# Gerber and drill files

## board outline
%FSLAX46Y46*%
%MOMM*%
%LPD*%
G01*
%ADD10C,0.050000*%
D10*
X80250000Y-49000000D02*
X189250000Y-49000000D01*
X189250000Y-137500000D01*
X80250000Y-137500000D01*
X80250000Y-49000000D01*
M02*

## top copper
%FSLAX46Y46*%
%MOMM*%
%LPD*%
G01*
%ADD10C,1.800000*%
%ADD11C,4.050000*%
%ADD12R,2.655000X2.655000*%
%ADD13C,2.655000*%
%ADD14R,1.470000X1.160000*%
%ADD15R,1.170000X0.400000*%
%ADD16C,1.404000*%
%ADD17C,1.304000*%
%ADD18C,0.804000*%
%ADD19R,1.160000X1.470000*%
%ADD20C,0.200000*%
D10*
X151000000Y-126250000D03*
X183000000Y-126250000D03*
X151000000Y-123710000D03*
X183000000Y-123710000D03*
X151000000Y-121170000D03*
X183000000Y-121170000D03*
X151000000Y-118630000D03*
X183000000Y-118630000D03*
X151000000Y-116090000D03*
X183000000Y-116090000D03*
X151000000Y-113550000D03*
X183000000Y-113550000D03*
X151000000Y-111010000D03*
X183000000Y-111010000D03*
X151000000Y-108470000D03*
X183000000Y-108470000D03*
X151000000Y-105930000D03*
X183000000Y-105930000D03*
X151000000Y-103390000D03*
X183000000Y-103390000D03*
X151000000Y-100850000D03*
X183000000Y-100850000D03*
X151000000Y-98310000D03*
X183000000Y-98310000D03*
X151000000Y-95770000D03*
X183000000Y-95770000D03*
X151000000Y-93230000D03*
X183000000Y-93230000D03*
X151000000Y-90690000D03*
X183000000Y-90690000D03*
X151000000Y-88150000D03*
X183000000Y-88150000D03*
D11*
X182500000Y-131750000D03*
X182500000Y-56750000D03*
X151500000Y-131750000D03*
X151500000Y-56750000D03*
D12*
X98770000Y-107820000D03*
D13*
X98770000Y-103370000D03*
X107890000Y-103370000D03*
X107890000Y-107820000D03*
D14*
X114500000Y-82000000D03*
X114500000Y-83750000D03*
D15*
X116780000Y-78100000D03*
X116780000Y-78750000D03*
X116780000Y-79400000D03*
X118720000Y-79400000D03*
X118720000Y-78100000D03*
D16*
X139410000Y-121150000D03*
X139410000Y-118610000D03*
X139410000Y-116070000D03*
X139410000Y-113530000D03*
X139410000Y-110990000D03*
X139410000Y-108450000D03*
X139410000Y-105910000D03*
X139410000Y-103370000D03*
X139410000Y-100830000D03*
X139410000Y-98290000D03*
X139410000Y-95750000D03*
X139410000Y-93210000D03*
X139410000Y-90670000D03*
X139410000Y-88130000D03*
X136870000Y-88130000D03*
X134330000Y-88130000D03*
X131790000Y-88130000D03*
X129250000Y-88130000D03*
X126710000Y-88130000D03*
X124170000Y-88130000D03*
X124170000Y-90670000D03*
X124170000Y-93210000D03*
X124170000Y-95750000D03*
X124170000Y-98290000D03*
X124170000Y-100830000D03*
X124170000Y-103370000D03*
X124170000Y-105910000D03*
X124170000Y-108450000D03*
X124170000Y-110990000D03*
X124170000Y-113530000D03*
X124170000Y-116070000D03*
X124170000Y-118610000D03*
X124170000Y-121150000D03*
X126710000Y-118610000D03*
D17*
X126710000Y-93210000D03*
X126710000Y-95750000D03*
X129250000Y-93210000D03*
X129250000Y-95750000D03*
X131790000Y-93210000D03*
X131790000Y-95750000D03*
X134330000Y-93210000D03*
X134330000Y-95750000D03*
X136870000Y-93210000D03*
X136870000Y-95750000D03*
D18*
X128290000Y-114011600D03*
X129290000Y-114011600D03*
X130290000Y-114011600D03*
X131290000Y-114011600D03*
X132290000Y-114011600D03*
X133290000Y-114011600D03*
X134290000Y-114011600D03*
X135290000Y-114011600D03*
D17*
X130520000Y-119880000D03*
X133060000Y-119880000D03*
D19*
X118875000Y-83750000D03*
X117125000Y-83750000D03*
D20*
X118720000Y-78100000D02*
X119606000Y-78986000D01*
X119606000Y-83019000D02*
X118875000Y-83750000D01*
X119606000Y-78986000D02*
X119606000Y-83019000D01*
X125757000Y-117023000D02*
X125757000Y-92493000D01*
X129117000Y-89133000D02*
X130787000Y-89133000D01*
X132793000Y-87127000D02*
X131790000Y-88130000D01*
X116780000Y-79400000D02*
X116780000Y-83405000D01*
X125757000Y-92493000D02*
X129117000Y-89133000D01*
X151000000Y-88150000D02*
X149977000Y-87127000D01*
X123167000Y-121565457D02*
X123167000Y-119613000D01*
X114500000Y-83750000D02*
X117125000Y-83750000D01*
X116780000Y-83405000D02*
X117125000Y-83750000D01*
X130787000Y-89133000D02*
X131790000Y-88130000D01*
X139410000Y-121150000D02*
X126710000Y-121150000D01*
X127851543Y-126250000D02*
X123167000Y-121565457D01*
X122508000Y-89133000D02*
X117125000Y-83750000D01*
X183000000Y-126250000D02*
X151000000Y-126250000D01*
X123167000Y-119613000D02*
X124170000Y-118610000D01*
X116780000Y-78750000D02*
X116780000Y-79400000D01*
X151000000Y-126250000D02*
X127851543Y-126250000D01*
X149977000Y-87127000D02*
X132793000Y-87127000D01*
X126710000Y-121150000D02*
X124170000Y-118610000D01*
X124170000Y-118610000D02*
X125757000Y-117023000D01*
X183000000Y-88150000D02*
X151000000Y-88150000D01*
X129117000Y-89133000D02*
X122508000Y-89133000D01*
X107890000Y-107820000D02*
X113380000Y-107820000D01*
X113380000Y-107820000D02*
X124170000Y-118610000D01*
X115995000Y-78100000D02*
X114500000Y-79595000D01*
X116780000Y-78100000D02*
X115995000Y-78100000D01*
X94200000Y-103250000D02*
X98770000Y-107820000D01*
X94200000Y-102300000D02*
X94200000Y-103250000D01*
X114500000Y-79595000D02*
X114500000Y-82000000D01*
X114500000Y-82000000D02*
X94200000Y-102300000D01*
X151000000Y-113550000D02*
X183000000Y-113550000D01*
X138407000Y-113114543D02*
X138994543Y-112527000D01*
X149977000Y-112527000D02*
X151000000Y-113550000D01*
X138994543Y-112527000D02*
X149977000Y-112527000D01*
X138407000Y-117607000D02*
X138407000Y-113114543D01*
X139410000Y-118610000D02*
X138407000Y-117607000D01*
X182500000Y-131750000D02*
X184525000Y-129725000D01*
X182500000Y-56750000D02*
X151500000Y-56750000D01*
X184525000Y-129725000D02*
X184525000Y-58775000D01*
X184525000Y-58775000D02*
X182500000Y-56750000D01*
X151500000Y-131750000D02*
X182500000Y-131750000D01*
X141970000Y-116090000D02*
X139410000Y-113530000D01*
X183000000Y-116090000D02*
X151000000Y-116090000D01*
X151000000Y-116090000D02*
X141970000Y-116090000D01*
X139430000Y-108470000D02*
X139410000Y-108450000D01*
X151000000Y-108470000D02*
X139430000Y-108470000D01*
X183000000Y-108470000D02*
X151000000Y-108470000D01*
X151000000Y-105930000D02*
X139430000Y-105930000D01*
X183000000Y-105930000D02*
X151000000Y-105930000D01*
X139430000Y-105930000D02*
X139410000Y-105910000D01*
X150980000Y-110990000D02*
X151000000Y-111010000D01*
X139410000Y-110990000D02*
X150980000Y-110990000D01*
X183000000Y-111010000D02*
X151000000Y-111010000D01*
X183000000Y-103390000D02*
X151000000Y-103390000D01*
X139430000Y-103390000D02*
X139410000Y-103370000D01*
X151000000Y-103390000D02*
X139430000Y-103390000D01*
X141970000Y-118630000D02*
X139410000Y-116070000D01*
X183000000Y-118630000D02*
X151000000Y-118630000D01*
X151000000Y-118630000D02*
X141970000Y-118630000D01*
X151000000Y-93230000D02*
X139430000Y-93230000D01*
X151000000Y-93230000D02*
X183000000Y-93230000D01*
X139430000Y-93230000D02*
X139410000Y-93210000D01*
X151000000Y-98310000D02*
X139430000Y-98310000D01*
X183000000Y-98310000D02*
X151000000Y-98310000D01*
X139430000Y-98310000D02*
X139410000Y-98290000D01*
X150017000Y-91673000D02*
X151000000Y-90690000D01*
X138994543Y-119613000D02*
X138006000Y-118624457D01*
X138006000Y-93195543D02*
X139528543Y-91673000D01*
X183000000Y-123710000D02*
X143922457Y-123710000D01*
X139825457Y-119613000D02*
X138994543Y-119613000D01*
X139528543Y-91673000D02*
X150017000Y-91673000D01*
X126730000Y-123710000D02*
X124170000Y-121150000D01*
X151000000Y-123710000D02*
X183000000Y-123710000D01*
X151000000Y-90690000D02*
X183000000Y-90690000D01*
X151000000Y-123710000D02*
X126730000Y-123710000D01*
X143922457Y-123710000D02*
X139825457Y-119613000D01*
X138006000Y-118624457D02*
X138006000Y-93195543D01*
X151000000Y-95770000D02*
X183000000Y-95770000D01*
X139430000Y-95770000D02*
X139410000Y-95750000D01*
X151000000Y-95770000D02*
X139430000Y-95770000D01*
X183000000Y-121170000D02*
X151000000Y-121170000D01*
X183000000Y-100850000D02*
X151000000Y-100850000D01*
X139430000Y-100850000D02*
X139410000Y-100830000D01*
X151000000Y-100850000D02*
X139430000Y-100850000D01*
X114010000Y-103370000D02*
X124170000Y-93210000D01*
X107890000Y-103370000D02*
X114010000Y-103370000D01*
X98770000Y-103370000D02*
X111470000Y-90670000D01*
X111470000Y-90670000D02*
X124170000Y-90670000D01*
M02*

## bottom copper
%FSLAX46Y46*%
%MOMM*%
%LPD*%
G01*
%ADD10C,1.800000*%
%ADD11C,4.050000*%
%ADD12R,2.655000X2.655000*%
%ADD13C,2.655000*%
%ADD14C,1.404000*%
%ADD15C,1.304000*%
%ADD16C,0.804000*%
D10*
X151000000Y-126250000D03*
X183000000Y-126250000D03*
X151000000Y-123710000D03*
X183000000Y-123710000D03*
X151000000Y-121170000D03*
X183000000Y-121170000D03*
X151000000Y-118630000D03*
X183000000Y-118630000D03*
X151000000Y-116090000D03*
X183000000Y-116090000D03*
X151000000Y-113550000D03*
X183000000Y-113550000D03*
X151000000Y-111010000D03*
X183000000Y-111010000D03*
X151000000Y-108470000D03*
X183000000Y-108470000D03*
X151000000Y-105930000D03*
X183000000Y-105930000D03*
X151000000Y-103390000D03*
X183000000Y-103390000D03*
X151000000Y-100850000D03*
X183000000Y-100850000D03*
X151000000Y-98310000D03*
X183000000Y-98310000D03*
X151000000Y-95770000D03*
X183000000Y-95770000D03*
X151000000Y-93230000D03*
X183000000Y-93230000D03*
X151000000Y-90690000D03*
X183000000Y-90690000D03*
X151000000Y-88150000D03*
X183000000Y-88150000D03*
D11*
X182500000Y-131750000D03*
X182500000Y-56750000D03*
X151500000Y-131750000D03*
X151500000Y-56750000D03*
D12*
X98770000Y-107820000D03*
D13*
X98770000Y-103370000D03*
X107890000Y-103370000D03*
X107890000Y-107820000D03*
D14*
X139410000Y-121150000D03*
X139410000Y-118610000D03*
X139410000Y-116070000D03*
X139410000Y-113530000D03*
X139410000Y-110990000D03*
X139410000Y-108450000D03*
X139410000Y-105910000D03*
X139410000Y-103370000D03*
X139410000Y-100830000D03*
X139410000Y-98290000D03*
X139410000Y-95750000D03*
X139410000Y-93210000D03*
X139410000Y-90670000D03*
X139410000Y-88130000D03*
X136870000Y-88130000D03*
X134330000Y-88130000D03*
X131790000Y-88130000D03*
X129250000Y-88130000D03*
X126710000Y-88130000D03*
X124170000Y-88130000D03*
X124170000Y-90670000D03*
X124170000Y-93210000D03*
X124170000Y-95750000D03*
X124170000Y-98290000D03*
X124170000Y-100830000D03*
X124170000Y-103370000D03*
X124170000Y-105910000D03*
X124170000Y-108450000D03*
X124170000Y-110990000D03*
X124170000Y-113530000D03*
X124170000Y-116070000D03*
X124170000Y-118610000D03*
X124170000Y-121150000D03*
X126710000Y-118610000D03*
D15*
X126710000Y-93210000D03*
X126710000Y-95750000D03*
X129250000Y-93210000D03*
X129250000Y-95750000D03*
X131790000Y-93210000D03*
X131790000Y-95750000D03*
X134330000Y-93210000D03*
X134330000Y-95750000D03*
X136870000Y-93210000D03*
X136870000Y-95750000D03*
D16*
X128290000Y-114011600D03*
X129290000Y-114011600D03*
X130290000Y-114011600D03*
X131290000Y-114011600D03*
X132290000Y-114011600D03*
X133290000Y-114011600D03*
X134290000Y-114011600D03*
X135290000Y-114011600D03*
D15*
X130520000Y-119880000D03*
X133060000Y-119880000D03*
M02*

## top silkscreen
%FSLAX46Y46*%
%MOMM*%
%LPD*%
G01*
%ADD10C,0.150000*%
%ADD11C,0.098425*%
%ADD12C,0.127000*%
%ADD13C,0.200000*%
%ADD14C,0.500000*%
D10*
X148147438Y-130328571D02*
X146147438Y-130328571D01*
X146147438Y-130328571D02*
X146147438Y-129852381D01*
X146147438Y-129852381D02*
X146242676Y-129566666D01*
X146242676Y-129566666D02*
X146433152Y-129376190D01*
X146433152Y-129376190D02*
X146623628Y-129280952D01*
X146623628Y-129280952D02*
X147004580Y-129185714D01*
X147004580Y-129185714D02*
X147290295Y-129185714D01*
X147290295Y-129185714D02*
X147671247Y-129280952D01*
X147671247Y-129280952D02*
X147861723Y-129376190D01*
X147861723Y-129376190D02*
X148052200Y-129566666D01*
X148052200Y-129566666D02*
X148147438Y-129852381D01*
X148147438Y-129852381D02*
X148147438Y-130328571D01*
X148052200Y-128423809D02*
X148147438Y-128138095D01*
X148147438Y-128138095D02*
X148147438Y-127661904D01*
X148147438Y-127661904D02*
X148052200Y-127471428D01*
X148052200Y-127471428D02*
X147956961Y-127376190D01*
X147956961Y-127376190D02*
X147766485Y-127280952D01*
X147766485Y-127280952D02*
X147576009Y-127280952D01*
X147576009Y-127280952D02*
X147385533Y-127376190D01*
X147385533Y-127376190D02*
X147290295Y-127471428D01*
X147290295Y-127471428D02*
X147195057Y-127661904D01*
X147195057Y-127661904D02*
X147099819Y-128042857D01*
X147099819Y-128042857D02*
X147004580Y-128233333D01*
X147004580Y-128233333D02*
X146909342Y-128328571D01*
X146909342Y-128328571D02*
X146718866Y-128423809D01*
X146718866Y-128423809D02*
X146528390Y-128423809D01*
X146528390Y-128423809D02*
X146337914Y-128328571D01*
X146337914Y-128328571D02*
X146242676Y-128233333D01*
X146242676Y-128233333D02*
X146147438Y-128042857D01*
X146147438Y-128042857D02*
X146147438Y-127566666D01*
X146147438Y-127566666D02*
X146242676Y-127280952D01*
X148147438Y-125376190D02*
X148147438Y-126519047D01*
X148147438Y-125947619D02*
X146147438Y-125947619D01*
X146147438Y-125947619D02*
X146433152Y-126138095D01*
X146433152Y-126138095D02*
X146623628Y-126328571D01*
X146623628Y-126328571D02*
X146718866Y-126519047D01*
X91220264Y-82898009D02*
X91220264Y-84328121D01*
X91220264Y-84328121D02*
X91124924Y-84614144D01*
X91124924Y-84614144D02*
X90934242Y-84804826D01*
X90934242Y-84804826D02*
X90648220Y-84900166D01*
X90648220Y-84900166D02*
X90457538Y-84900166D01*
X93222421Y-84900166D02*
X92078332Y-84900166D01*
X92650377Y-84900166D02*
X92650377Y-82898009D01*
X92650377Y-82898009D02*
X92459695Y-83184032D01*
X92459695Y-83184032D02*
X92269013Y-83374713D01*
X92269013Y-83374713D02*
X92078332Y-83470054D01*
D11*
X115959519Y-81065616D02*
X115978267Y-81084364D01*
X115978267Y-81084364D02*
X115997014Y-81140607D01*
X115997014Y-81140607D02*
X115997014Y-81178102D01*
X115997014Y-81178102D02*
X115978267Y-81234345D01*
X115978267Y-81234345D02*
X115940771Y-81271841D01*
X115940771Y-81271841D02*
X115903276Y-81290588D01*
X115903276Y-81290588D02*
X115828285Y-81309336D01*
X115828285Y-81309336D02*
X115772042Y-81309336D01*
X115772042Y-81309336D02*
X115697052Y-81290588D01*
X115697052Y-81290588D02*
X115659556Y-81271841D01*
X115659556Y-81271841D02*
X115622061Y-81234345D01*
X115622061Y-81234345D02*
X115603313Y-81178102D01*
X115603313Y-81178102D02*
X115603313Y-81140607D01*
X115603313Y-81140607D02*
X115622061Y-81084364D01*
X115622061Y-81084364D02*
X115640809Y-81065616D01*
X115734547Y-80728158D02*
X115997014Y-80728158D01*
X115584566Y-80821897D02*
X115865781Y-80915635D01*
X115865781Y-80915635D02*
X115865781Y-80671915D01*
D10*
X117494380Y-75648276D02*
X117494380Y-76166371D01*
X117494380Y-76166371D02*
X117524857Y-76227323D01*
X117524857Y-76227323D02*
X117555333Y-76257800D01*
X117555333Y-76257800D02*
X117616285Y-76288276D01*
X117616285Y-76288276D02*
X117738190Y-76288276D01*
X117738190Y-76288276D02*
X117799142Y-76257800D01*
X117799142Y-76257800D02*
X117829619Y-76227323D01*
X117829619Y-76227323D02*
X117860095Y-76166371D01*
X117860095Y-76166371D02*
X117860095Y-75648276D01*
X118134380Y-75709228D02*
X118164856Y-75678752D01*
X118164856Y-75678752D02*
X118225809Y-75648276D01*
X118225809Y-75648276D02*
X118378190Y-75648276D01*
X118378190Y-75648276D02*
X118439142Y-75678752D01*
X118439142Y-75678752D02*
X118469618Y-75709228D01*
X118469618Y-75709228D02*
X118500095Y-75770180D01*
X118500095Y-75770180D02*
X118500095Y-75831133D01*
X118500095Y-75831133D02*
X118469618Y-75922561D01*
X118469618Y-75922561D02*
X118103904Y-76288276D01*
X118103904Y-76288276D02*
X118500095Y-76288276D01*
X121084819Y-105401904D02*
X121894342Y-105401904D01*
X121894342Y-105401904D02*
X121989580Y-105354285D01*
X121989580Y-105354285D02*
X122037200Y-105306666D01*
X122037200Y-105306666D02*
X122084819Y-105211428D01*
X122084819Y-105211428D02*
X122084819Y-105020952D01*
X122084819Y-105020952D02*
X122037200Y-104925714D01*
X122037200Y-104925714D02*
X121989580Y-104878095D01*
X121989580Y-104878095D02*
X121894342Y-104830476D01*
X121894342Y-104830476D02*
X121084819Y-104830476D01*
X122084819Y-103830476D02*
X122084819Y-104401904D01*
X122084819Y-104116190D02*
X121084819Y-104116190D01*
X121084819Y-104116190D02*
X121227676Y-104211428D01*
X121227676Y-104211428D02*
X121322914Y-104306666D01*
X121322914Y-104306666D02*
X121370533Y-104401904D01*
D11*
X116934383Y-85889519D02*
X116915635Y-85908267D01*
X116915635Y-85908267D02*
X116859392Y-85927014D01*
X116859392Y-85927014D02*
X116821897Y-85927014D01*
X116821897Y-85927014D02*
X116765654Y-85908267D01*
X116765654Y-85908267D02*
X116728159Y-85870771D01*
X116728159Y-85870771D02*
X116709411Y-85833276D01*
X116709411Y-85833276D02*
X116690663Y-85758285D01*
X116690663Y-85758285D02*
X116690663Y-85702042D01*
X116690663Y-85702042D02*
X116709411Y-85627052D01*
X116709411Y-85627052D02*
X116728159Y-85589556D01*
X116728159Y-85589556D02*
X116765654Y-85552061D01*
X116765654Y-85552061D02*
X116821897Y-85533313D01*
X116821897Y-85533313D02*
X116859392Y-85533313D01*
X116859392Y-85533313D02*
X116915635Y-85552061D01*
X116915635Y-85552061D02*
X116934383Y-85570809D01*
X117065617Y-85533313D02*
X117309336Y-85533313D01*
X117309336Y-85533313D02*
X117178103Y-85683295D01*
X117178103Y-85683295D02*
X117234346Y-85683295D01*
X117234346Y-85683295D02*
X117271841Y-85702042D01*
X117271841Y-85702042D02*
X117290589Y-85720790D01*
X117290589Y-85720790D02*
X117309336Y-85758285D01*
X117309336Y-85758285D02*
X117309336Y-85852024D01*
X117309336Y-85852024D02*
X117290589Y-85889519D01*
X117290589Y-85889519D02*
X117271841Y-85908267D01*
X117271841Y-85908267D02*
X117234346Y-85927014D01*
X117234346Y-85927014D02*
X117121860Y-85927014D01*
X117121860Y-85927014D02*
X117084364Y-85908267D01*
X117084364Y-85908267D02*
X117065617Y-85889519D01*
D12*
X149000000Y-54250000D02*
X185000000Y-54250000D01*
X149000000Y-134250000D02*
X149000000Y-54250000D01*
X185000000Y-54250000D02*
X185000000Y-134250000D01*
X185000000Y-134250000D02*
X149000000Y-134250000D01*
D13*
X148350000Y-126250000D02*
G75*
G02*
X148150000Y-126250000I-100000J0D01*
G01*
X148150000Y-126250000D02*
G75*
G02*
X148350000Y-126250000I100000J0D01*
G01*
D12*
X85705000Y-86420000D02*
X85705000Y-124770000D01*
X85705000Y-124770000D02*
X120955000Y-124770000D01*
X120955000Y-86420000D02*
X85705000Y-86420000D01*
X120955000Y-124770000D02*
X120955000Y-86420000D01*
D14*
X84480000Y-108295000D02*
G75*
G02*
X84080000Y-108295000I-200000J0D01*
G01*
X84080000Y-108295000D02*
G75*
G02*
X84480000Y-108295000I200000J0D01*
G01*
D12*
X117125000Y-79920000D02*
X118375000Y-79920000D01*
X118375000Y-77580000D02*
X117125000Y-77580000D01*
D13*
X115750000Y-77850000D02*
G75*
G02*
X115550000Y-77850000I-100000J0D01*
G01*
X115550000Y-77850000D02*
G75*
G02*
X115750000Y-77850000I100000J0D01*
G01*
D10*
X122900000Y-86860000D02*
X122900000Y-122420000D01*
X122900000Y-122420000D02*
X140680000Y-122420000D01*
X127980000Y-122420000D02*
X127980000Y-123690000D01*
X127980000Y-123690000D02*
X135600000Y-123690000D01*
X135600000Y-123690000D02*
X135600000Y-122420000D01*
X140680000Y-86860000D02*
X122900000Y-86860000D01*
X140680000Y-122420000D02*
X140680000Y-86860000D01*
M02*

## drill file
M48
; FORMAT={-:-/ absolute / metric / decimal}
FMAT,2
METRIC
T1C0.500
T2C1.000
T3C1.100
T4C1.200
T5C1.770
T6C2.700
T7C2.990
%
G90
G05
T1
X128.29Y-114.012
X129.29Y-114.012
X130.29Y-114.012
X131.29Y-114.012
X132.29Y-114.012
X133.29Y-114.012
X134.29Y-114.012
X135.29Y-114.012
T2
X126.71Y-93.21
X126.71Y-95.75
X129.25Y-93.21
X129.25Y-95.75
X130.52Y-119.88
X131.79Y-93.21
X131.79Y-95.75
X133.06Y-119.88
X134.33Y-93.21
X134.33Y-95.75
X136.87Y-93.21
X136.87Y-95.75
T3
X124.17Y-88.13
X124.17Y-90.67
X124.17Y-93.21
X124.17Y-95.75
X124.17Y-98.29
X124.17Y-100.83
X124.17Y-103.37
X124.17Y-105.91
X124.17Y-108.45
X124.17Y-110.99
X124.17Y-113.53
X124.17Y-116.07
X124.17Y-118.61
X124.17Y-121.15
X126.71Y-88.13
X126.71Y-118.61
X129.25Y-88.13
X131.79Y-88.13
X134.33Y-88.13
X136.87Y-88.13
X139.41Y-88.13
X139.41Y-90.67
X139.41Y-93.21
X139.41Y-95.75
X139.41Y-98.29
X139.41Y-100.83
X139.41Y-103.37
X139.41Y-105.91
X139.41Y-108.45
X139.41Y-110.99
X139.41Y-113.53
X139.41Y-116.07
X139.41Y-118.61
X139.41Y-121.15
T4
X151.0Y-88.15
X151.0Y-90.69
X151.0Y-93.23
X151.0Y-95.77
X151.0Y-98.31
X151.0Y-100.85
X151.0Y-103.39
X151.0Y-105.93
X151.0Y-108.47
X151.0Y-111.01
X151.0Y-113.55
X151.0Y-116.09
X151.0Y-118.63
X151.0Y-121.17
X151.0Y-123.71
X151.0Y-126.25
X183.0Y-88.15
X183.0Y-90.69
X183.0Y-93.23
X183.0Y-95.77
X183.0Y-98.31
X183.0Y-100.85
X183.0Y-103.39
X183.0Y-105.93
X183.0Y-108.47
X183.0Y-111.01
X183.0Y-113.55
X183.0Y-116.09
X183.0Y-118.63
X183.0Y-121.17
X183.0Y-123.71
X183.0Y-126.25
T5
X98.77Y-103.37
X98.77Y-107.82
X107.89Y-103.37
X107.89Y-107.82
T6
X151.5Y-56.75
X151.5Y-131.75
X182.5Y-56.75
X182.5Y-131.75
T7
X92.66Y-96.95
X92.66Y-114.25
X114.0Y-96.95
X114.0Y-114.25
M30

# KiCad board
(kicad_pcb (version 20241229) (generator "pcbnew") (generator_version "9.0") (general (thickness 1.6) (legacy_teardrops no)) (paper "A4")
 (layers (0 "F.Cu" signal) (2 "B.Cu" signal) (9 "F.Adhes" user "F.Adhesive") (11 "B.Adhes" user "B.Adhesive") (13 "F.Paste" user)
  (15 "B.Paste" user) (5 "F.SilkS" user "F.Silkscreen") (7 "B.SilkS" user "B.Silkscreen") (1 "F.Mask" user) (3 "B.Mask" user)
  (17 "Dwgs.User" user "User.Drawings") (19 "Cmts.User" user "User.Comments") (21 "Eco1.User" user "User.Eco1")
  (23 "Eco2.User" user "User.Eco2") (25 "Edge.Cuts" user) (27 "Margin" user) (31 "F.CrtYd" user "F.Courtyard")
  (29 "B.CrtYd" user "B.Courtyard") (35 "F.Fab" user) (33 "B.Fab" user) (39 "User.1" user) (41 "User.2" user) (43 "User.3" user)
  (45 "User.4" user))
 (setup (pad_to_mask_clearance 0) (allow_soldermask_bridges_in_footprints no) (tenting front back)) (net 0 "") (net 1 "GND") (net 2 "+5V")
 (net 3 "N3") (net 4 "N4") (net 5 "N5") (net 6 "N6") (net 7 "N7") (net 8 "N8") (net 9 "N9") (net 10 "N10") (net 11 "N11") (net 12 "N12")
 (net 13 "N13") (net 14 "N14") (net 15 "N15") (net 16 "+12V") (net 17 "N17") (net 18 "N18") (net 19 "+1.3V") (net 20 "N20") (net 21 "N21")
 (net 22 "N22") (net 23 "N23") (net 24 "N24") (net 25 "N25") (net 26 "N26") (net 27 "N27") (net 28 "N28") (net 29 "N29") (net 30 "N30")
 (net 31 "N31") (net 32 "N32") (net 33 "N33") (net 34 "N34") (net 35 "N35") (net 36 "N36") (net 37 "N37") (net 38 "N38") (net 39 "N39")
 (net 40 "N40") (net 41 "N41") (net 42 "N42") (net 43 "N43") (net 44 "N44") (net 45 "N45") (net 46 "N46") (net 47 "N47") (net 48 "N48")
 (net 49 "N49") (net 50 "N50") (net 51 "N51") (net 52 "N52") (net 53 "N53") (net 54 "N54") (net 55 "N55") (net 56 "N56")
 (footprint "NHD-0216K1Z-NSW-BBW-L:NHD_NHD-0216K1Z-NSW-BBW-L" (layer "F.Cu") (at 167 94.25 90)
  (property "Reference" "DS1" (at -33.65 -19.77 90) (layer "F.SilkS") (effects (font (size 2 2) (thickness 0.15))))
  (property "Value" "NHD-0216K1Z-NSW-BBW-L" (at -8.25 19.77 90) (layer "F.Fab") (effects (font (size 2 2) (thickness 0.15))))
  (fp_line (start 40 -18) (end 40 18) (stroke (width 0.127) (type solid)) (layer "F.SilkS"))
  (fp_line (start -40 -18) (end 40 -18) (stroke (width 0.127) (type solid)) (layer "F.SilkS"))
  (fp_line (start 40 18) (end -40 18) (stroke (width 0.127) (type solid)) (layer "F.SilkS"))
  (fp_line (start -40 18) (end -40 -18) (stroke (width 0.127) (type solid)) (layer "F.SilkS"))
  (fp_circle (center -32 -18.75) (end -31.9 -18.75) (stroke (width 0.2) (type solid)) (fill no) (layer "F.SilkS"))
  (pad "1_1" thru_hole circle (at -32 -16 90) (size 1.8 1.8) (drill 1.2) (layers "*.Cu" "*.Mask") (remove_unused_layers no) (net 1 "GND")
   (solder_mask_margin 0.102))
  (pad "1_2" thru_hole circle (at -32 16 90) (size 1.8 1.8) (drill 1.2) (layers "*.Cu" "*.Mask") (remove_unused_layers no) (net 1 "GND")
   (solder_mask_margin 0.102))
  (pad "2_1" thru_hole circle (at -29.46 -16 90) (size 1.8 1.8) (drill 1.2) (layers "*.Cu" "*.Mask") (remove_unused_layers no) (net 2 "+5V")
   (solder_mask_margin 0.102))
  (pad "2_2" thru_hole circle (at -29.46 16 90) (size 1.8 1.8) (drill 1.2) (layers "*.Cu" "*.Mask") (remove_unused_layers no) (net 2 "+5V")
   (solder_mask_margin 0.102))
  (pad "3_1" thru_hole circle (at -26.92 -16 90) (size 1.8 1.8) (drill 1.2) (layers "*.Cu" "*.Mask") (remove_unused_layers no) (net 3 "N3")
   (solder_mask_margin 0.102))
  (pad "3_2" thru_hole circle (at -26.92 16 90) (size 1.8 1.8) (drill 1.2) (layers "*.Cu" "*.Mask") (remove_unused_layers no) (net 3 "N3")
   (solder_mask_margin 0.102))
  (pad "4_1" thru_hole circle (at -24.38 -16 90) (size 1.8 1.8) (drill 1.2) (layers "*.Cu" "*.Mask") (remove_unused_layers no) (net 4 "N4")
   (solder_mask_margin 0.102))
  (pad "4_2" thru_hole circle (at -24.38 16 90) (size 1.8 1.8) (drill 1.2) (layers "*.Cu" "*.Mask") (remove_unused_layers no) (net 4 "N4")
   (solder_mask_margin 0.102))
  (pad "5_1" thru_hole circle (at -21.84 -16 90) (size 1.8 1.8) (drill 1.2) (layers "*.Cu" "*.Mask") (remove_unused_layers no) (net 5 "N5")
   (solder_mask_margin 0.102))
  (pad "5_2" thru_hole circle (at -21.84 16 90) (size 1.8 1.8) (drill 1.2) (layers "*.Cu" "*.Mask") (remove_unused_layers no) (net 5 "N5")
   (solder_mask_margin 0.102))
  (pad "6_1" thru_hole circle (at -19.3 -16 90) (size 1.8 1.8) (drill 1.2) (layers "*.Cu" "*.Mask") (remove_unused_layers no) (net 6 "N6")
   (solder_mask_margin 0.102))
  (pad "6_2" thru_hole circle (at -19.3 16 90) (size 1.8 1.8) (drill 1.2) (layers "*.Cu" "*.Mask") (remove_unused_layers no) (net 6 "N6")
   (solder_mask_margin 0.102))
  (pad "7_1" thru_hole circle (at -16.76 -16 90) (size 1.8 1.8) (drill 1.2) (layers "*.Cu" "*.Mask") (remove_unused_layers no) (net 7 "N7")
   (solder_mask_margin 0.102))
  (pad "7_2" thru_hole circle (at -16.76 16 90) (size 1.8 1.8) (drill 1.2) (layers "*.Cu" "*.Mask") (remove_unused_layers no) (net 7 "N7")
   (solder_mask_margin 0.102))
  (pad "8_1" thru_hole circle (at -14.22 -16 90) (size 1.8 1.8) (drill 1.2) (layers "*.Cu" "*.Mask") (remove_unused_layers no) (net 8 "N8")
   (solder_mask_margin 0.102))
  (pad "8_2" thru_hole circle (at -14.22 16 90) (size 1.8 1.8) (drill 1.2) (layers "*.Cu" "*.Mask") (remove_unused_layers no) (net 8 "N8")
   (solder_mask_margin 0.102))
  (pad "9_1" thru_hole circle (at -11.68 -16 90) (size 1.8 1.8) (drill 1.2) (layers "*.Cu" "*.Mask") (remove_unused_layers no) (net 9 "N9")
   (solder_mask_margin 0.102))
  (pad "9_2" thru_hole circle (at -11.68 16 90) (size 1.8 1.8) (drill 1.2) (layers "*.Cu" "*.Mask") (remove_unused_layers no) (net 9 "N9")
   (solder_mask_margin 0.102))
  (pad "10_1" thru_hole circle (at -9.14 -16 90) (size 1.8 1.8) (drill 1.2) (layers "*.Cu" "*.Mask") (remove_unused_layers no)
   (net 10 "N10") (solder_mask_margin 0.102))
  (pad "10_2" thru_hole circle (at -9.14 16 90) (size 1.8 1.8) (drill 1.2) (layers "*.Cu" "*.Mask") (remove_unused_layers no) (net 10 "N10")
   (solder_mask_margin 0.102))
  (pad "11_1" thru_hole circle (at -6.6 -16 90) (size 1.8 1.8) (drill 1.2) (layers "*.Cu" "*.Mask") (remove_unused_layers no) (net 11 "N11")
   (solder_mask_margin 0.102))
  (pad "11_2" thru_hole circle (at -6.6 16 90) (size 1.8 1.8) (drill 1.2) (layers "*.Cu" "*.Mask") (remove_unused_layers no) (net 11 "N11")
   (solder_mask_margin 0.102))
  (pad "12_1" thru_hole circle (at -4.06 -16 90) (size 1.8 1.8) (drill 1.2) (layers "*.Cu" "*.Mask") (remove_unused_layers no)
   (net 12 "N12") (solder_mask_margin 0.102))
  (pad "12_2" thru_hole circle (at -4.06 16 90) (size 1.8 1.8) (drill 1.2) (layers "*.Cu" "*.Mask") (remove_unused_layers no) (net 12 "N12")
   (solder_mask_margin 0.102))
  (pad "13_1" thru_hole circle (at -1.52 -16 90) (size 1.8 1.8) (drill 1.2) (layers "*.Cu" "*.Mask") (remove_unused_layers no)
   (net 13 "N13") (solder_mask_margin 0.102))
  (pad "13_2" thru_hole circle (at -1.52 16 90) (size 1.8 1.8) (drill 1.2) (layers "*.Cu" "*.Mask") (remove_unused_layers no) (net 13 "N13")
   (solder_mask_margin 0.102))
  (pad "14_1" thru_hole circle (at 1.02 -16 90) (size 1.8 1.8) (drill 1.2) (layers "*.Cu" "*.Mask") (remove_unused_layers no) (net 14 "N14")
   (solder_mask_margin 0.102))
  (pad "14_2" thru_hole circle (at 1.02 16 90) (size 1.8 1.8) (drill 1.2) (layers "*.Cu" "*.Mask") (remove_unused_layers no) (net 14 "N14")
   (solder_mask_margin 0.102))
  (pad "15_1" thru_hole circle (at 3.56 -16 90) (size 1.8 1.8) (drill 1.2) (layers "*.Cu" "*.Mask") (remove_unused_layers no) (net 2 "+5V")
   (solder_mask_margin 0.102))
  (pad "15_2" thru_hole circle (at 3.56 16 90) (size 1.8 1.8) (drill 1.2) (layers "*.Cu" "*.Mask") (remove_unused_layers no) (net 2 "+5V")
   (solder_mask_margin 0.102))
  (pad "16_1" thru_hole circle (at 6.1 -16 90) (size 1.8 1.8) (drill 1.2) (layers "*.Cu" "*.Mask") (remove_unused_layers no) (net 1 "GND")
   (solder_mask_margin 0.102))
  (pad "16_2" thru_hole circle (at 6.1 16 90) (size 1.8 1.8) (drill 1.2) (layers "*.Cu" "*.Mask") (remove_unused_layers no) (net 1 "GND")
   (solder_mask_margin 0.102))
  (pad "S1" thru_hole circle (at -37.5 15.5 90) (size 4.05 4.05) (drill 2.7) (layers "*.Cu" "*.Mask") (remove_unused_layers no)
   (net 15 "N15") (solder_mask_margin 0.102))
  (pad "S2" thru_hole circle (at 37.5 15.5 90) (size 4.05 4.05) (drill 2.7) (layers "*.Cu" "*.Mask") (remove_unused_layers no)
   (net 15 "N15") (solder_mask_margin 0.102))
  (pad "S3" thru_hole circle (at -37.5 -15.5 90) (size 4.05 4.05) (drill 2.7) (layers "*.Cu" "*.Mask") (remove_unused_layers no)
   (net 15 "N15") (solder_mask_margin 0.102))
  (pad "S4" thru_hole circle (at 37.5 -15.5 90) (size 4.05 4.05) (drill 2.7) (layers "*.Cu" "*.Mask") (remove_unused_layers no)
   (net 15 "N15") (solder_mask_margin 0.102)))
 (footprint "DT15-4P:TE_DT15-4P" (layer "F.Cu") (at 103.33 105.595)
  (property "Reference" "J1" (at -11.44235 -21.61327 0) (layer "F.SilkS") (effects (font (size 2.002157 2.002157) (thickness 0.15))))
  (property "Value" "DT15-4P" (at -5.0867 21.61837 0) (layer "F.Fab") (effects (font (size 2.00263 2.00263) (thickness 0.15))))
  (fp_line (start -17.625 -19.175) (end -17.625 19.175) (stroke (width 0.127) (type solid)) (layer "F.SilkS"))
  (fp_line (start -17.625 19.175) (end 17.625 19.175) (stroke (width 0.127) (type solid)) (layer "F.SilkS"))
  (fp_line (start 17.625 -19.175) (end -17.625 -19.175) (stroke (width 0.127) (type solid)) (layer "F.SilkS"))
  (fp_line (start 17.625 19.175) (end 17.625 -19.175) (stroke (width 0.127) (type solid)) (layer "F.SilkS"))
  (fp_circle (center -19.05 2.7) (end -18.85 2.7) (stroke (width 0.5) (type solid)) (fill no) (layer "F.SilkS"))
  (pad "" np_thru_hole circle (at -10.67 -8.645) (size 2.99 2.99) (drill 2.99) (layers "*.Cu" "*.Mask"))
  (pad "" np_thru_hole circle (at -10.67 8.655) (size 2.99 2.99) (drill 2.99) (layers "*.Cu" "*.Mask"))
  (pad "" np_thru_hole circle (at 10.67 -8.645) (size 2.99 2.99) (drill 2.99) (layers "*.Cu" "*.Mask"))
  (pad "" np_thru_hole circle (at 10.67 8.655) (size 2.99 2.99) (drill 2.99) (layers "*.Cu" "*.Mask"))
  (pad "1" thru_hole rect (at -4.56 2.225) (size 2.655 2.655) (drill 1.77) (layers "*.Cu" "*.Mask") (remove_unused_layers no)
   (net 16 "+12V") (solder_mask_margin 0.102))
  (pad "2" thru_hole circle (at -4.56 -2.225) (size 2.655 2.655) (drill 1.77) (layers "*.Cu" "*.Mask") (remove_unused_layers no)
   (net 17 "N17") (solder_mask_margin 0.102))
  (pad "3" thru_hole circle (at 4.56 -2.225) (size 2.655 2.655) (drill 1.77) (layers "*.Cu" "*.Mask") (remove_unused_layers no)
   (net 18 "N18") (solder_mask_margin 0.102))
  (pad "4" thru_hole circle (at 4.56 2.225) (size 2.655 2.655) (drill 1.77) (layers "*.Cu" "*.Mask") (remove_unused_layers no) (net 1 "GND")
   (solder_mask_margin 0.102)))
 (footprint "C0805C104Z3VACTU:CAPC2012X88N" (layer "F.Cu") (at 114.5 82.875 -90)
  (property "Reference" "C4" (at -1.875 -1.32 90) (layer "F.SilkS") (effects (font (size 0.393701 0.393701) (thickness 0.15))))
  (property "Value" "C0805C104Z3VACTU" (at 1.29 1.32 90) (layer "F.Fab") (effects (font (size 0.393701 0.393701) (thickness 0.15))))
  (pad "1" smd rect (at -0.875 0 270) (size 1.16 1.47) (layers "F.Cu" "F.Mask" "F.Paste") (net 16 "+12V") (solder_mask_margin 0.102))
  (pad "2" smd rect (at 0.875 0 270) (size 1.16 1.47) (layers "F.Cu" "F.Mask" "F.Paste") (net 1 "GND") (solder_mask_margin 0.102)))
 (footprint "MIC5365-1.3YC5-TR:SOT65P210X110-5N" (layer "F.Cu") (at 117.75 78.75)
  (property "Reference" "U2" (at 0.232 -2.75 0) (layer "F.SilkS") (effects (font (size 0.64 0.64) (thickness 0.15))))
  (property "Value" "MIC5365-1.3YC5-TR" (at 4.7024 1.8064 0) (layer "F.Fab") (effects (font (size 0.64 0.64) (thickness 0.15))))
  (fp_line (start -0.625 1.17) (end 0.625 1.17) (stroke (width 0.127) (type solid)) (layer "F.SilkS"))
  (fp_line (start 0.625 -1.17) (end -0.625 -1.17) (stroke (width 0.127) (type solid)) (layer "F.SilkS"))
  (fp_circle (center -2.1 -0.9) (end -2 -0.9) (stroke (width 0.2) (type solid)) (fill no) (layer "F.SilkS"))
  (pad "1" smd rect (at -0.97 -0.65) (size 1.17 0.4) (layers "F.Cu" "F.Mask" "F.Paste") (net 16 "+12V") (solder_mask_margin 0.102))
  (pad "2" smd rect (at -0.97 0) (size 1.17 0.4) (layers "F.Cu" "F.Mask" "F.Paste") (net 1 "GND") (solder_mask_margin 0.102))
  (pad "3" smd rect (at -0.97 0.65) (size 1.17 0.4) (layers "F.Cu" "F.Mask" "F.Paste") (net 1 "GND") (solder_mask_margin 0.102))
  (pad "4" smd rect (at 0.97 0.65) (size 1.17 0.4) (layers "F.Cu" "F.Mask" "F.Paste") (solder_mask_margin 0.102))
  (pad "5" smd rect (at 0.97 -0.65) (size 1.17 0.4) (layers "F.Cu" "F.Mask" "F.Paste") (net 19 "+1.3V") (solder_mask_margin 0.102)))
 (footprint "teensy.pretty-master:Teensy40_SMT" (layer "F.Cu") (at 131.79 104.64 90)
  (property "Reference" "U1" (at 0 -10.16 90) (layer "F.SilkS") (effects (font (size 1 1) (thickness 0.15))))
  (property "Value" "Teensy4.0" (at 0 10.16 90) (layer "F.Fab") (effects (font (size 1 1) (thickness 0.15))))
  (fp_line (start 17.78 -8.89) (end -17.78 -8.89) (stroke (width 0.15) (type solid)) (layer "F.SilkS"))
  (fp_line (start -17.78 -8.89) (end -17.78 8.89) (stroke (width 0.15) (type solid)) (layer "F.SilkS"))
  (fp_line (start -17.78 -3.81) (end -19.05 -3.81) (stroke (width 0.15) (type solid)) (layer "F.SilkS"))
  (fp_line (start -19.05 -3.81) (end -19.05 3.81) (stroke (width 0.15) (type solid)) (layer "F.SilkS"))
  (fp_line (start -19.05 3.81) (end -17.78 3.81) (stroke (width 0.15) (type solid)) (layer "F.SilkS"))
  (fp_line (start 17.78 8.89) (end 17.78 -8.89) (stroke (width 0.15) (type solid)) (layer "F.SilkS"))
  (fp_line (start -17.78 8.89) (end 17.78 8.89) (stroke (width 0.15) (type solid)) (layer "F.SilkS"))
  (pad "1" thru_hole circle (at -16.51 7.62 90) (size 1.404 1.404) (drill 1.1) (layers "*.Cu" "*.Mask") (remove_unused_layers no)
   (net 1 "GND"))
  (pad "2" thru_hole circle (at -13.97 7.62 90) (size 1.404 1.404) (drill 1.1) (layers "*.Cu" "*.Mask") (remove_unused_layers no)
   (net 6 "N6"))
  (pad "3" thru_hole circle (at -11.43 7.62 90) (size 1.404 1.404) (drill 1.1) (layers "*.Cu" "*.Mask") (remove_unused_layers no)
   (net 4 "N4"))
  (pad "4" thru_hole circle (at -8.89 7.62 90) (size 1.404 1.404) (drill 1.1) (layers "*.Cu" "*.Mask") (remove_unused_layers no)
   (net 5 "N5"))
  (pad "5" thru_hole circle (at -6.35 7.62 90) (size 1.404 1.404) (drill 1.1) (layers "*.Cu" "*.Mask") (remove_unused_layers no)
   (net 7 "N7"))
  (pad "6" thru_hole circle (at -3.81 7.62 90) (size 1.404 1.404) (drill 1.1) (layers "*.Cu" "*.Mask") (remove_unused_layers no)
   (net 8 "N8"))
  (pad "7" thru_hole circle (at -1.27 7.62 90) (size 1.404 1.404) (drill 1.1) (layers "*.Cu" "*.Mask") (remove_unused_layers no)
   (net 9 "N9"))
  (pad "8" thru_hole circle (at 1.27 7.62 90) (size 1.404 1.404) (drill 1.1) (layers "*.Cu" "*.Mask") (remove_unused_layers no)
   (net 10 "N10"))
  (pad "9" thru_hole circle (at 3.81 7.62 90) (size 1.404 1.404) (drill 1.1) (layers "*.Cu" "*.Mask") (remove_unused_layers no)
   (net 11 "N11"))
  (pad "10" thru_hole circle (at 6.35 7.62 90) (size 1.404 1.404) (drill 1.1) (layers "*.Cu" "*.Mask") (remove_unused_layers no)
   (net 12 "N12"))
  (pad "11" thru_hole circle (at 8.89 7.62 90) (size 1.404 1.404) (drill 1.1) (layers "*.Cu" "*.Mask") (remove_unused_layers no)
   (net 13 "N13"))
  (pad "12" thru_hole circle (at 11.43 7.62 90) (size 1.404 1.404) (drill 1.1) (layers "*.Cu" "*.Mask") (remove_unused_layers no)
   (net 14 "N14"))
  (pad "13" thru_hole circle (at 13.97 7.62 90) (size 1.404 1.404) (drill 1.1) (layers "*.Cu" "*.Mask") (remove_unused_layers no)
   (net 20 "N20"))
  (pad "14" thru_hole circle (at 16.51 7.62 90) (size 1.404 1.404) (drill 1.1) (layers "*.Cu" "*.Mask") (remove_unused_layers no)
   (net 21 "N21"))
  (pad "15" thru_hole circle (at 16.51 5.08 90) (size 1.404 1.404) (drill 1.1) (layers "*.Cu" "*.Mask") (remove_unused_layers no)
   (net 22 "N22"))
  (pad "16" thru_hole circle (at 16.51 2.54 90) (size 1.404 1.404) (drill 1.1) (layers "*.Cu" "*.Mask") (remove_unused_layers no)
   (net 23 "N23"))
  (pad "17" thru_hole circle (at 16.51 0 90) (size 1.404 1.404) (drill 1.1) (layers "*.Cu" "*.Mask") (remove_unused_layers no) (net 1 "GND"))
  (pad "18" thru_hole circle (at 16.51 -2.54 90) (size 1.404 1.404) (drill 1.1) (layers "*.Cu" "*.Mask") (remove_unused_layers no)
   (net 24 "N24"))
  (pad "19" thru_hole circle (at 16.51 -5.08 90) (size 1.404 1.404) (drill 1.1) (layers "*.Cu" "*.Mask") (remove_unused_layers no)
   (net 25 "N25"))
  (pad "20" thru_hole circle (at 16.51 -7.62 90) (size 1.404 1.404) (drill 1.1) (layers "*.Cu" "*.Mask") (remove_unused_layers no)
   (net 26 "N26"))
  (pad "21" thru_hole circle (at 13.97 -7.62 90) (size 1.404 1.404) (drill 1.1) (layers "*.Cu" "*.Mask") (remove_unused_layers no)
   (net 17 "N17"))
  (pad "22" thru_hole circle (at 11.43 -7.62 90) (size 1.404 1.404) (drill 1.1) (layers "*.Cu" "*.Mask") (remove_unused_layers no)
   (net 18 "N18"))
  (pad "23" thru_hole circle (at 8.89 -7.62 90) (size 1.404 1.404) (drill 1.1) (layers "*.Cu" "*.Mask") (remove_unused_layers no)
   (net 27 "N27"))
  (pad "24" thru_hole circle (at 6.35 -7.62 90) (size 1.404 1.404) (drill 1.1) (layers "*.Cu" "*.Mask") (remove_unused_layers no)
   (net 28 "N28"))
  (pad "25" thru_hole circle (at 3.81 -7.62 90) (size 1.404 1.404) (drill 1.1) (layers "*.Cu" "*.Mask") (remove_unused_layers no)
   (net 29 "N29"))
  (pad "26" thru_hole circle (at 1.27 -7.62 90) (size 1.404 1.404) (drill 1.1) (layers "*.Cu" "*.Mask") (remove_unused_layers no)
   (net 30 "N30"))
  (pad "27" thru_hole circle (at -1.27 -7.62 90) (size 1.404 1.404) (drill 1.1) (layers "*.Cu" "*.Mask") (remove_unused_layers no)
   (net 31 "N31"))
  (pad "28" thru_hole circle (at -3.81 -7.62 90) (size 1.404 1.404) (drill 1.1) (layers "*.Cu" "*.Mask") (remove_unused_layers no)
   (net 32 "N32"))
  (pad "29" thru_hole circle (at -6.35 -7.62 90) (size 1.404 1.404) (drill 1.1) (layers "*.Cu" "*.Mask") (remove_unused_layers no)
   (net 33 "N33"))
  (pad "30" thru_hole circle (at -8.89 -7.62 90) (size 1.404 1.404) (drill 1.1) (layers "*.Cu" "*.Mask") (remove_unused_layers no)
   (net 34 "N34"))
  (pad "31" thru_hole circle (at -11.43 -7.62 90) (size 1.404 1.404) (drill 1.1) (layers "*.Cu" "*.Mask") (remove_unused_layers no)
   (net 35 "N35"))
  (pad "32" thru_hole circle (at -13.97 -7.62 90) (size 1.404 1.404) (drill 1.1) (layers "*.Cu" "*.Mask") (remove_unused_layers no)
   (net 1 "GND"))
  (pad "33" thru_hole circle (at -16.51 -7.62 90) (size 1.404 1.404) (drill 1.1) (layers "*.Cu" "*.Mask") (remove_unused_layers no)
   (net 2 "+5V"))
  (pad "34" thru_hole circle (at -13.97 -5.08 90) (size 1.404 1.404) (drill 1.1) (layers "*.Cu" "*.Mask") (remove_unused_layers no)
   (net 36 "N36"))
  (pad "35" thru_hole circle (at 11.43 -5.08 90) (size 1.304 1.304) (drill 1) (layers "*.Cu" "*.Mask") (remove_unused_layers no)
   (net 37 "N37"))
  (pad "36" thru_hole circle (at 8.89 -5.08 90) (size 1.304 1.304) (drill 1) (layers "*.Cu" "*.Mask") (remove_unused_layers no)
   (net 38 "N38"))
  (pad "37" thru_hole circle (at 11.43 -2.54 90) (size 1.304 1.304) (drill 1) (layers "*.Cu" "*.Mask") (remove_unused_layers no)
   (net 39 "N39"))
  (pad "38" thru_hole circle (at 8.89 -2.54 90) (size 1.304 1.304) (drill 1) (layers "*.Cu" "*.Mask") (remove_unused_layers no)
   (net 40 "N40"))
  (pad "39" thru_hole circle (at 11.43 0 90) (size 1.304 1.304) (drill 1) (layers "*.Cu" "*.Mask") (remove_unused_layers no) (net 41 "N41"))
  (pad "40" thru_hole circle (at 8.89 0 90) (size 1.304 1.304) (drill 1) (layers "*.Cu" "*.Mask") (remove_unused_layers no) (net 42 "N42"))
  (pad "41" thru_hole circle (at 11.43 2.54 90) (size 1.304 1.304) (drill 1) (layers "*.Cu" "*.Mask") (remove_unused_layers no)
   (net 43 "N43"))
  (pad "42" thru_hole circle (at 8.89 2.54 90) (size 1.304 1.304) (drill 1) (layers "*.Cu" "*.Mask") (remove_unused_layers no)
   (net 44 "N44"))
  (pad "43" thru_hole circle (at 11.43 5.08 90) (size 1.304 1.304) (drill 1) (layers "*.Cu" "*.Mask") (remove_unused_layers no)
   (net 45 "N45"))
  (pad "44" thru_hole circle (at 8.89 5.08 90) (size 1.304 1.304) (drill 1) (layers "*.Cu" "*.Mask") (remove_unused_layers no)
   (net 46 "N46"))
  (pad "45" thru_hole circle (at -9.3716 -3.5 90) (size 0.804 0.804) (drill 0.5) (layers "*.Cu" "*.Mask") (remove_unused_layers no)
   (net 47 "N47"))
  (pad "46" thru_hole circle (at -9.3716 -2.5 90) (size 0.804 0.804) (drill 0.5) (layers "*.Cu" "*.Mask") (remove_unused_layers no)
   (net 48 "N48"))
  (pad "47" thru_hole circle (at -9.3716 -1.5 90) (size 0.804 0.804) (drill 0.5) (layers "*.Cu" "*.Mask") (remove_unused_layers no)
   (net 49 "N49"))
  (pad "48" thru_hole circle (at -9.3716 -0.5 90) (size 0.804 0.804) (drill 0.5) (layers "*.Cu" "*.Mask") (remove_unused_layers no)
   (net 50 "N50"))
  (pad "49" thru_hole circle (at -9.3716 0.5 90) (size 0.804 0.804) (drill 0.5) (layers "*.Cu" "*.Mask") (remove_unused_layers no)
   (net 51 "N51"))
  (pad "50" thru_hole circle (at -9.3716 1.5 90) (size 0.804 0.804) (drill 0.5) (layers "*.Cu" "*.Mask") (remove_unused_layers no)
   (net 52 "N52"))
  (pad "51" thru_hole circle (at -9.3716 2.5 90) (size 0.804 0.804) (drill 0.5) (layers "*.Cu" "*.Mask") (remove_unused_layers no)
   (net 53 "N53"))
  (pad "52" thru_hole circle (at -9.3716 3.5 90) (size 0.804 0.804) (drill 0.5) (layers "*.Cu" "*.Mask") (remove_unused_layers no)
   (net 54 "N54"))
  (pad "53" thru_hole circle (at -15.24 -1.27 90) (size 1.304 1.304) (drill 1) (layers "*.Cu" "*.Mask") (remove_unused_layers no)
   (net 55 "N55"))
  (pad "54" thru_hole circle (at -15.24 1.27 90) (size 1.304 1.304) (drill 1) (layers "*.Cu" "*.Mask") (remove_unused_layers no)
   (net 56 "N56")))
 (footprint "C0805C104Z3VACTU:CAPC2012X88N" (layer "F.Cu") (at 118 83.75 180)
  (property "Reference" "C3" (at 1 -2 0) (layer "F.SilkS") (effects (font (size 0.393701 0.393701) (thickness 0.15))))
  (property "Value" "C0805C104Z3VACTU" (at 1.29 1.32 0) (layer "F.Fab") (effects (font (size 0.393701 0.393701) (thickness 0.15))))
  (pad "1" smd rect (at -0.875 0 180) (size 1.16 1.47) (layers "F.Cu" "F.Mask" "F.Paste") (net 19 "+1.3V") (solder_mask_margin 0.102))
  (pad "2" smd rect (at 0.875 0 180) (size 1.16 1.47) (layers "F.Cu" "F.Mask" "F.Paste") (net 1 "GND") (solder_mask_margin 0.102)))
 (gr_rect (start 80.25 49) (end 189.25 137.5) (stroke (width 0.05) (type default)) (fill no) (layer "Edge.Cuts"))
 (segment (start 118.72 78.1) (end 119.606 78.986) (width 0.2) (layer "F.Cu") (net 19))
 (segment (start 119.606 83.019) (end 118.875 83.75) (width 0.2) (layer "F.Cu") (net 19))
 (segment (start 119.606 78.986) (end 119.606 83.019) (width 0.2) (layer "F.Cu") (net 19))
 (segment (start 125.757 117.023) (end 125.757 92.493) (width 0.2) (layer "F.Cu") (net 1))
 (segment (start 129.117 89.133) (end 130.787 89.133) (width 0.2) (layer "F.Cu") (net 1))
 (segment (start 132.793 87.127) (end 131.79 88.13) (width 0.2) (layer "F.Cu") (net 1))
 (segment (start 116.78 79.4) (end 116.78 83.405) (width 0.2) (layer "F.Cu") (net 1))
 (segment (start 125.757 92.493) (end 129.117 89.133) (width 0.2) (layer "F.Cu") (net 1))
 (segment (start 151 88.15) (end 149.977 87.127) (width 0.2) (layer "F.Cu") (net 1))
 (segment (start 123.167 121.565457) (end 123.167 119.613) (width 0.2) (layer "F.Cu") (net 1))
 (segment (start 114.5 83.75) (end 117.125 83.75) (width 0.2) (layer "F.Cu") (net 1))
 (segment (start 116.78 83.405) (end 117.125 83.75) (width 0.2) (layer "F.Cu") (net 1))
 (segment (start 130.787 89.133) (end 131.79 88.13) (width 0.2) (layer "F.Cu") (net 1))
 (segment (start 139.41 121.15) (end 126.71 121.15) (width 0.2) (layer "F.Cu") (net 1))
 (segment (start 127.851543 126.25) (end 123.167 121.565457) (width 0.2) (layer "F.Cu") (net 1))
 (segment (start 122.508 89.133) (end 117.125 83.75) (width 0.2) (layer "F.Cu") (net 1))
 (segment (start 183 126.25) (end 151 126.25) (width 0.2) (layer "F.Cu") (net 1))
 (segment (start 123.167 119.613) (end 124.17 118.61) (width 0.2) (layer "F.Cu") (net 1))
 (segment (start 116.78 78.75) (end 116.78 79.4) (width 0.2) (layer "F.Cu") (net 1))
 (segment (start 151 126.25) (end 127.851543 126.25) (width 0.2) (layer "F.Cu") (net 1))
 (segment (start 149.977 87.127) (end 132.793 87.127) (width 0.2) (layer "F.Cu") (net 1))
 (segment (start 126.71 121.15) (end 124.17 118.61) (width 0.2) (layer "F.Cu") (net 1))
 (segment (start 124.17 118.61) (end 125.757 117.023) (width 0.2) (layer "F.Cu") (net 1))
 (segment (start 183 88.15) (end 151 88.15) (width 0.2) (layer "F.Cu") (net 1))
 (segment (start 129.117 89.133) (end 122.508 89.133) (width 0.2) (layer "F.Cu") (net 1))
 (segment (start 107.89 107.82) (end 113.38 107.82) (width 0.2) (layer "F.Cu") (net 1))
 (segment (start 113.38 107.82) (end 124.17 118.61) (width 0.2) (layer "F.Cu") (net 1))
 (segment (start 115.995 78.1) (end 114.5 79.595) (width 0.2) (layer "F.Cu") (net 16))
 (segment (start 116.78 78.1) (end 115.995 78.1) (width 0.2) (layer "F.Cu") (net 16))
 (segment (start 94.2 103.25) (end 98.77 107.82) (width 0.2) (layer "F.Cu") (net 16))
 (segment (start 94.2 102.3) (end 94.2 103.25) (width 0.2) (layer "F.Cu") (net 16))
 (segment (start 114.5 79.595) (end 114.5 82) (width 0.2) (layer "F.Cu") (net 16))
 (segment (start 114.5 82) (end 94.2 102.3) (width 0.2) (layer "F.Cu") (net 16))
 (segment (start 151 113.55) (end 183 113.55) (width 0.2) (layer "F.Cu") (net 6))
 (segment (start 138.407 113.114543) (end 138.994543 112.527) (width 0.2) (layer "F.Cu") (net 6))
 (segment (start 149.977 112.527) (end 151 113.55) (width 0.2) (layer "F.Cu") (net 6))
 (segment (start 138.994543 112.527) (end 149.977 112.527) (width 0.2) (layer "F.Cu") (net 6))
 (segment (start 138.407 117.607) (end 138.407 113.114543) (width 0.2) (layer "F.Cu") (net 6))
 (segment (start 139.41 118.61) (end 138.407 117.607) (width 0.2) (layer "F.Cu") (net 6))
 (segment (start 182.5 131.75) (end 184.525 129.725) (width 0.2) (layer "F.Cu") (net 15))
 (segment (start 182.5 56.75) (end 151.5 56.75) (width 0.2) (layer "F.Cu") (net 15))
 (segment (start 184.525 129.725) (end 184.525 58.775) (width 0.2) (layer "F.Cu") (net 15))
 (segment (start 184.525 58.775) (end 182.5 56.75) (width 0.2) (layer "F.Cu") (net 15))
 (segment (start 151.5 131.75) (end 182.5 131.75) (width 0.2) (layer "F.Cu") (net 15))
 (segment (start 141.97 116.09) (end 139.41 113.53) (width 0.2) (layer "F.Cu") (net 5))
 (segment (start 183 116.09) (end 151 116.09) (width 0.2) (layer "F.Cu") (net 5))
 (segment (start 151 116.09) (end 141.97 116.09) (width 0.2) (layer "F.Cu") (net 5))
 (segment (start 139.43 108.47) (end 139.41 108.45) (width 0.2) (layer "F.Cu") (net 8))
 (segment (start 151 108.47) (end 139.43 108.47) (width 0.2) (layer "F.Cu") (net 8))
 (segment (start 183 108.47) (end 151 108.47) (width 0.2) (layer "F.Cu") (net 8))
 (segment (start 151 105.93) (end 139.43 105.93) (width 0.2) (layer "F.Cu") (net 9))
 (segment (start 183 105.93) (end 151 105.93) (width 0.2) (layer "F.Cu") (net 9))
 (segment (start 139.43 105.93) (end 139.41 105.91) (width 0.2) (layer "F.Cu") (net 9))
 (segment (start 150.98 110.99) (end 151 111.01) (width 0.2) (layer "F.Cu") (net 7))
 (segment (start 139.41 110.99) (end 150.98 110.99) (width 0.2) (layer "F.Cu") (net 7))
 (segment (start 183 111.01) (end 151 111.01) (width 0.2) (layer "F.Cu") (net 7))
 (segment (start 183 103.39) (end 151 103.39) (width 0.2) (layer "F.Cu") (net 10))
 (segment (start 139.43 103.39) (end 139.41 103.37) (width 0.2) (layer "F.Cu") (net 10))
 (segment (start 151 103.39) (end 139.43 103.39) (width 0.2) (layer "F.Cu") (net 10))
 (segment (start 141.97 118.63) (end 139.41 116.07) (width 0.2) (layer "F.Cu") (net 4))
 (segment (start 183 118.63) (end 151 118.63) (width 0.2) (layer "F.Cu") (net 4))
 (segment (start 151 118.63) (end 141.97 118.63) (width 0.2) (layer "F.Cu") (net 4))
 (segment (start 151 93.23) (end 139.43 93.23) (width 0.2) (layer "F.Cu") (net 14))
 (segment (start 151 93.23) (end 183 93.23) (width 0.2) (layer "F.Cu") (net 14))
 (segment (start 139.43 93.23) (end 139.41 93.21) (width 0.2) (layer "F.Cu") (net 14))
 (segment (start 151 98.31) (end 139.43 98.31) (width 0.2) (layer "F.Cu") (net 12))
 (segment (start 183 98.31) (end 151 98.31) (width 0.2) (layer "F.Cu") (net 12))
 (segment (start 139.43 98.31) (end 139.41 98.29) (width 0.2) (layer "F.Cu") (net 12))
 (segment (start 150.017 91.673) (end 151 90.69) (width 0.2) (layer "F.Cu") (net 2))
 (segment (start 138.994543 119.613) (end 138.006 118.624457) (width 0.2) (layer "F.Cu") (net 2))
 (segment (start 138.006 93.195543) (end 139.528543 91.673) (width 0.2) (layer "F.Cu") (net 2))
 (segment (start 183 123.71) (end 143.922457 123.71) (width 0.2) (layer "F.Cu") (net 2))
 (segment (start 139.825457 119.613) (end 138.994543 119.613) (width 0.2) (layer "F.Cu") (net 2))
 (segment (start 139.528543 91.673) (end 150.017 91.673) (width 0.2) (layer "F.Cu") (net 2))
 (segment (start 126.73 123.71) (end 124.17 121.15) (width 0.2) (layer "F.Cu") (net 2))
 (segment (start 151 123.71) (end 183 123.71) (width 0.2) (layer "F.Cu") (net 2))
 (segment (start 151 90.69) (end 183 90.69) (width 0.2) (layer "F.Cu") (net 2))
 (segment (start 151 123.71) (end 126.73 123.71) (width 0.2) (layer "F.Cu") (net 2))
 (segment (start 143.922457 123.71) (end 139.825457 119.613) (width 0.2) (layer "F.Cu") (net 2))
 (segment (start 138.006 118.624457) (end 138.006 93.195543) (width 0.2) (layer "F.Cu") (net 2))
 (segment (start 151 95.77) (end 183 95.77) (width 0.2) (layer "F.Cu") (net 13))
 (segment (start 139.43 95.77) (end 139.41 95.75) (width 0.2) (layer "F.Cu") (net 13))
 (segment (start 151 95.77) (end 139.43 95.77) (width 0.2) (layer "F.Cu") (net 13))
 (segment (start 183 121.17) (end 151 121.17) (width 0.2) (layer "F.Cu") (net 3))
 (segment (start 183 100.85) (end 151 100.85) (width 0.2) (layer "F.Cu") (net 11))
 (segment (start 139.43 100.85) (end 139.41 100.83) (width 0.2) (layer "F.Cu") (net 11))
 (segment (start 151 100.85) (end 139.43 100.85) (width 0.2) (layer "F.Cu") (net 11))
 (segment (start 114.01 103.37) (end 124.17 93.21) (width 0.2) (layer "F.Cu") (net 18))
 (segment (start 107.89 103.37) (end 114.01 103.37) (width 0.2) (layer "F.Cu") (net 18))
 (segment (start 98.77 103.37) (end 111.47 90.67) (width 0.2) (layer "F.Cu") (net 17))
 (segment (start 111.47 90.67) (end 124.17 90.67) (width 0.2) (layer "F.Cu") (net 17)))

